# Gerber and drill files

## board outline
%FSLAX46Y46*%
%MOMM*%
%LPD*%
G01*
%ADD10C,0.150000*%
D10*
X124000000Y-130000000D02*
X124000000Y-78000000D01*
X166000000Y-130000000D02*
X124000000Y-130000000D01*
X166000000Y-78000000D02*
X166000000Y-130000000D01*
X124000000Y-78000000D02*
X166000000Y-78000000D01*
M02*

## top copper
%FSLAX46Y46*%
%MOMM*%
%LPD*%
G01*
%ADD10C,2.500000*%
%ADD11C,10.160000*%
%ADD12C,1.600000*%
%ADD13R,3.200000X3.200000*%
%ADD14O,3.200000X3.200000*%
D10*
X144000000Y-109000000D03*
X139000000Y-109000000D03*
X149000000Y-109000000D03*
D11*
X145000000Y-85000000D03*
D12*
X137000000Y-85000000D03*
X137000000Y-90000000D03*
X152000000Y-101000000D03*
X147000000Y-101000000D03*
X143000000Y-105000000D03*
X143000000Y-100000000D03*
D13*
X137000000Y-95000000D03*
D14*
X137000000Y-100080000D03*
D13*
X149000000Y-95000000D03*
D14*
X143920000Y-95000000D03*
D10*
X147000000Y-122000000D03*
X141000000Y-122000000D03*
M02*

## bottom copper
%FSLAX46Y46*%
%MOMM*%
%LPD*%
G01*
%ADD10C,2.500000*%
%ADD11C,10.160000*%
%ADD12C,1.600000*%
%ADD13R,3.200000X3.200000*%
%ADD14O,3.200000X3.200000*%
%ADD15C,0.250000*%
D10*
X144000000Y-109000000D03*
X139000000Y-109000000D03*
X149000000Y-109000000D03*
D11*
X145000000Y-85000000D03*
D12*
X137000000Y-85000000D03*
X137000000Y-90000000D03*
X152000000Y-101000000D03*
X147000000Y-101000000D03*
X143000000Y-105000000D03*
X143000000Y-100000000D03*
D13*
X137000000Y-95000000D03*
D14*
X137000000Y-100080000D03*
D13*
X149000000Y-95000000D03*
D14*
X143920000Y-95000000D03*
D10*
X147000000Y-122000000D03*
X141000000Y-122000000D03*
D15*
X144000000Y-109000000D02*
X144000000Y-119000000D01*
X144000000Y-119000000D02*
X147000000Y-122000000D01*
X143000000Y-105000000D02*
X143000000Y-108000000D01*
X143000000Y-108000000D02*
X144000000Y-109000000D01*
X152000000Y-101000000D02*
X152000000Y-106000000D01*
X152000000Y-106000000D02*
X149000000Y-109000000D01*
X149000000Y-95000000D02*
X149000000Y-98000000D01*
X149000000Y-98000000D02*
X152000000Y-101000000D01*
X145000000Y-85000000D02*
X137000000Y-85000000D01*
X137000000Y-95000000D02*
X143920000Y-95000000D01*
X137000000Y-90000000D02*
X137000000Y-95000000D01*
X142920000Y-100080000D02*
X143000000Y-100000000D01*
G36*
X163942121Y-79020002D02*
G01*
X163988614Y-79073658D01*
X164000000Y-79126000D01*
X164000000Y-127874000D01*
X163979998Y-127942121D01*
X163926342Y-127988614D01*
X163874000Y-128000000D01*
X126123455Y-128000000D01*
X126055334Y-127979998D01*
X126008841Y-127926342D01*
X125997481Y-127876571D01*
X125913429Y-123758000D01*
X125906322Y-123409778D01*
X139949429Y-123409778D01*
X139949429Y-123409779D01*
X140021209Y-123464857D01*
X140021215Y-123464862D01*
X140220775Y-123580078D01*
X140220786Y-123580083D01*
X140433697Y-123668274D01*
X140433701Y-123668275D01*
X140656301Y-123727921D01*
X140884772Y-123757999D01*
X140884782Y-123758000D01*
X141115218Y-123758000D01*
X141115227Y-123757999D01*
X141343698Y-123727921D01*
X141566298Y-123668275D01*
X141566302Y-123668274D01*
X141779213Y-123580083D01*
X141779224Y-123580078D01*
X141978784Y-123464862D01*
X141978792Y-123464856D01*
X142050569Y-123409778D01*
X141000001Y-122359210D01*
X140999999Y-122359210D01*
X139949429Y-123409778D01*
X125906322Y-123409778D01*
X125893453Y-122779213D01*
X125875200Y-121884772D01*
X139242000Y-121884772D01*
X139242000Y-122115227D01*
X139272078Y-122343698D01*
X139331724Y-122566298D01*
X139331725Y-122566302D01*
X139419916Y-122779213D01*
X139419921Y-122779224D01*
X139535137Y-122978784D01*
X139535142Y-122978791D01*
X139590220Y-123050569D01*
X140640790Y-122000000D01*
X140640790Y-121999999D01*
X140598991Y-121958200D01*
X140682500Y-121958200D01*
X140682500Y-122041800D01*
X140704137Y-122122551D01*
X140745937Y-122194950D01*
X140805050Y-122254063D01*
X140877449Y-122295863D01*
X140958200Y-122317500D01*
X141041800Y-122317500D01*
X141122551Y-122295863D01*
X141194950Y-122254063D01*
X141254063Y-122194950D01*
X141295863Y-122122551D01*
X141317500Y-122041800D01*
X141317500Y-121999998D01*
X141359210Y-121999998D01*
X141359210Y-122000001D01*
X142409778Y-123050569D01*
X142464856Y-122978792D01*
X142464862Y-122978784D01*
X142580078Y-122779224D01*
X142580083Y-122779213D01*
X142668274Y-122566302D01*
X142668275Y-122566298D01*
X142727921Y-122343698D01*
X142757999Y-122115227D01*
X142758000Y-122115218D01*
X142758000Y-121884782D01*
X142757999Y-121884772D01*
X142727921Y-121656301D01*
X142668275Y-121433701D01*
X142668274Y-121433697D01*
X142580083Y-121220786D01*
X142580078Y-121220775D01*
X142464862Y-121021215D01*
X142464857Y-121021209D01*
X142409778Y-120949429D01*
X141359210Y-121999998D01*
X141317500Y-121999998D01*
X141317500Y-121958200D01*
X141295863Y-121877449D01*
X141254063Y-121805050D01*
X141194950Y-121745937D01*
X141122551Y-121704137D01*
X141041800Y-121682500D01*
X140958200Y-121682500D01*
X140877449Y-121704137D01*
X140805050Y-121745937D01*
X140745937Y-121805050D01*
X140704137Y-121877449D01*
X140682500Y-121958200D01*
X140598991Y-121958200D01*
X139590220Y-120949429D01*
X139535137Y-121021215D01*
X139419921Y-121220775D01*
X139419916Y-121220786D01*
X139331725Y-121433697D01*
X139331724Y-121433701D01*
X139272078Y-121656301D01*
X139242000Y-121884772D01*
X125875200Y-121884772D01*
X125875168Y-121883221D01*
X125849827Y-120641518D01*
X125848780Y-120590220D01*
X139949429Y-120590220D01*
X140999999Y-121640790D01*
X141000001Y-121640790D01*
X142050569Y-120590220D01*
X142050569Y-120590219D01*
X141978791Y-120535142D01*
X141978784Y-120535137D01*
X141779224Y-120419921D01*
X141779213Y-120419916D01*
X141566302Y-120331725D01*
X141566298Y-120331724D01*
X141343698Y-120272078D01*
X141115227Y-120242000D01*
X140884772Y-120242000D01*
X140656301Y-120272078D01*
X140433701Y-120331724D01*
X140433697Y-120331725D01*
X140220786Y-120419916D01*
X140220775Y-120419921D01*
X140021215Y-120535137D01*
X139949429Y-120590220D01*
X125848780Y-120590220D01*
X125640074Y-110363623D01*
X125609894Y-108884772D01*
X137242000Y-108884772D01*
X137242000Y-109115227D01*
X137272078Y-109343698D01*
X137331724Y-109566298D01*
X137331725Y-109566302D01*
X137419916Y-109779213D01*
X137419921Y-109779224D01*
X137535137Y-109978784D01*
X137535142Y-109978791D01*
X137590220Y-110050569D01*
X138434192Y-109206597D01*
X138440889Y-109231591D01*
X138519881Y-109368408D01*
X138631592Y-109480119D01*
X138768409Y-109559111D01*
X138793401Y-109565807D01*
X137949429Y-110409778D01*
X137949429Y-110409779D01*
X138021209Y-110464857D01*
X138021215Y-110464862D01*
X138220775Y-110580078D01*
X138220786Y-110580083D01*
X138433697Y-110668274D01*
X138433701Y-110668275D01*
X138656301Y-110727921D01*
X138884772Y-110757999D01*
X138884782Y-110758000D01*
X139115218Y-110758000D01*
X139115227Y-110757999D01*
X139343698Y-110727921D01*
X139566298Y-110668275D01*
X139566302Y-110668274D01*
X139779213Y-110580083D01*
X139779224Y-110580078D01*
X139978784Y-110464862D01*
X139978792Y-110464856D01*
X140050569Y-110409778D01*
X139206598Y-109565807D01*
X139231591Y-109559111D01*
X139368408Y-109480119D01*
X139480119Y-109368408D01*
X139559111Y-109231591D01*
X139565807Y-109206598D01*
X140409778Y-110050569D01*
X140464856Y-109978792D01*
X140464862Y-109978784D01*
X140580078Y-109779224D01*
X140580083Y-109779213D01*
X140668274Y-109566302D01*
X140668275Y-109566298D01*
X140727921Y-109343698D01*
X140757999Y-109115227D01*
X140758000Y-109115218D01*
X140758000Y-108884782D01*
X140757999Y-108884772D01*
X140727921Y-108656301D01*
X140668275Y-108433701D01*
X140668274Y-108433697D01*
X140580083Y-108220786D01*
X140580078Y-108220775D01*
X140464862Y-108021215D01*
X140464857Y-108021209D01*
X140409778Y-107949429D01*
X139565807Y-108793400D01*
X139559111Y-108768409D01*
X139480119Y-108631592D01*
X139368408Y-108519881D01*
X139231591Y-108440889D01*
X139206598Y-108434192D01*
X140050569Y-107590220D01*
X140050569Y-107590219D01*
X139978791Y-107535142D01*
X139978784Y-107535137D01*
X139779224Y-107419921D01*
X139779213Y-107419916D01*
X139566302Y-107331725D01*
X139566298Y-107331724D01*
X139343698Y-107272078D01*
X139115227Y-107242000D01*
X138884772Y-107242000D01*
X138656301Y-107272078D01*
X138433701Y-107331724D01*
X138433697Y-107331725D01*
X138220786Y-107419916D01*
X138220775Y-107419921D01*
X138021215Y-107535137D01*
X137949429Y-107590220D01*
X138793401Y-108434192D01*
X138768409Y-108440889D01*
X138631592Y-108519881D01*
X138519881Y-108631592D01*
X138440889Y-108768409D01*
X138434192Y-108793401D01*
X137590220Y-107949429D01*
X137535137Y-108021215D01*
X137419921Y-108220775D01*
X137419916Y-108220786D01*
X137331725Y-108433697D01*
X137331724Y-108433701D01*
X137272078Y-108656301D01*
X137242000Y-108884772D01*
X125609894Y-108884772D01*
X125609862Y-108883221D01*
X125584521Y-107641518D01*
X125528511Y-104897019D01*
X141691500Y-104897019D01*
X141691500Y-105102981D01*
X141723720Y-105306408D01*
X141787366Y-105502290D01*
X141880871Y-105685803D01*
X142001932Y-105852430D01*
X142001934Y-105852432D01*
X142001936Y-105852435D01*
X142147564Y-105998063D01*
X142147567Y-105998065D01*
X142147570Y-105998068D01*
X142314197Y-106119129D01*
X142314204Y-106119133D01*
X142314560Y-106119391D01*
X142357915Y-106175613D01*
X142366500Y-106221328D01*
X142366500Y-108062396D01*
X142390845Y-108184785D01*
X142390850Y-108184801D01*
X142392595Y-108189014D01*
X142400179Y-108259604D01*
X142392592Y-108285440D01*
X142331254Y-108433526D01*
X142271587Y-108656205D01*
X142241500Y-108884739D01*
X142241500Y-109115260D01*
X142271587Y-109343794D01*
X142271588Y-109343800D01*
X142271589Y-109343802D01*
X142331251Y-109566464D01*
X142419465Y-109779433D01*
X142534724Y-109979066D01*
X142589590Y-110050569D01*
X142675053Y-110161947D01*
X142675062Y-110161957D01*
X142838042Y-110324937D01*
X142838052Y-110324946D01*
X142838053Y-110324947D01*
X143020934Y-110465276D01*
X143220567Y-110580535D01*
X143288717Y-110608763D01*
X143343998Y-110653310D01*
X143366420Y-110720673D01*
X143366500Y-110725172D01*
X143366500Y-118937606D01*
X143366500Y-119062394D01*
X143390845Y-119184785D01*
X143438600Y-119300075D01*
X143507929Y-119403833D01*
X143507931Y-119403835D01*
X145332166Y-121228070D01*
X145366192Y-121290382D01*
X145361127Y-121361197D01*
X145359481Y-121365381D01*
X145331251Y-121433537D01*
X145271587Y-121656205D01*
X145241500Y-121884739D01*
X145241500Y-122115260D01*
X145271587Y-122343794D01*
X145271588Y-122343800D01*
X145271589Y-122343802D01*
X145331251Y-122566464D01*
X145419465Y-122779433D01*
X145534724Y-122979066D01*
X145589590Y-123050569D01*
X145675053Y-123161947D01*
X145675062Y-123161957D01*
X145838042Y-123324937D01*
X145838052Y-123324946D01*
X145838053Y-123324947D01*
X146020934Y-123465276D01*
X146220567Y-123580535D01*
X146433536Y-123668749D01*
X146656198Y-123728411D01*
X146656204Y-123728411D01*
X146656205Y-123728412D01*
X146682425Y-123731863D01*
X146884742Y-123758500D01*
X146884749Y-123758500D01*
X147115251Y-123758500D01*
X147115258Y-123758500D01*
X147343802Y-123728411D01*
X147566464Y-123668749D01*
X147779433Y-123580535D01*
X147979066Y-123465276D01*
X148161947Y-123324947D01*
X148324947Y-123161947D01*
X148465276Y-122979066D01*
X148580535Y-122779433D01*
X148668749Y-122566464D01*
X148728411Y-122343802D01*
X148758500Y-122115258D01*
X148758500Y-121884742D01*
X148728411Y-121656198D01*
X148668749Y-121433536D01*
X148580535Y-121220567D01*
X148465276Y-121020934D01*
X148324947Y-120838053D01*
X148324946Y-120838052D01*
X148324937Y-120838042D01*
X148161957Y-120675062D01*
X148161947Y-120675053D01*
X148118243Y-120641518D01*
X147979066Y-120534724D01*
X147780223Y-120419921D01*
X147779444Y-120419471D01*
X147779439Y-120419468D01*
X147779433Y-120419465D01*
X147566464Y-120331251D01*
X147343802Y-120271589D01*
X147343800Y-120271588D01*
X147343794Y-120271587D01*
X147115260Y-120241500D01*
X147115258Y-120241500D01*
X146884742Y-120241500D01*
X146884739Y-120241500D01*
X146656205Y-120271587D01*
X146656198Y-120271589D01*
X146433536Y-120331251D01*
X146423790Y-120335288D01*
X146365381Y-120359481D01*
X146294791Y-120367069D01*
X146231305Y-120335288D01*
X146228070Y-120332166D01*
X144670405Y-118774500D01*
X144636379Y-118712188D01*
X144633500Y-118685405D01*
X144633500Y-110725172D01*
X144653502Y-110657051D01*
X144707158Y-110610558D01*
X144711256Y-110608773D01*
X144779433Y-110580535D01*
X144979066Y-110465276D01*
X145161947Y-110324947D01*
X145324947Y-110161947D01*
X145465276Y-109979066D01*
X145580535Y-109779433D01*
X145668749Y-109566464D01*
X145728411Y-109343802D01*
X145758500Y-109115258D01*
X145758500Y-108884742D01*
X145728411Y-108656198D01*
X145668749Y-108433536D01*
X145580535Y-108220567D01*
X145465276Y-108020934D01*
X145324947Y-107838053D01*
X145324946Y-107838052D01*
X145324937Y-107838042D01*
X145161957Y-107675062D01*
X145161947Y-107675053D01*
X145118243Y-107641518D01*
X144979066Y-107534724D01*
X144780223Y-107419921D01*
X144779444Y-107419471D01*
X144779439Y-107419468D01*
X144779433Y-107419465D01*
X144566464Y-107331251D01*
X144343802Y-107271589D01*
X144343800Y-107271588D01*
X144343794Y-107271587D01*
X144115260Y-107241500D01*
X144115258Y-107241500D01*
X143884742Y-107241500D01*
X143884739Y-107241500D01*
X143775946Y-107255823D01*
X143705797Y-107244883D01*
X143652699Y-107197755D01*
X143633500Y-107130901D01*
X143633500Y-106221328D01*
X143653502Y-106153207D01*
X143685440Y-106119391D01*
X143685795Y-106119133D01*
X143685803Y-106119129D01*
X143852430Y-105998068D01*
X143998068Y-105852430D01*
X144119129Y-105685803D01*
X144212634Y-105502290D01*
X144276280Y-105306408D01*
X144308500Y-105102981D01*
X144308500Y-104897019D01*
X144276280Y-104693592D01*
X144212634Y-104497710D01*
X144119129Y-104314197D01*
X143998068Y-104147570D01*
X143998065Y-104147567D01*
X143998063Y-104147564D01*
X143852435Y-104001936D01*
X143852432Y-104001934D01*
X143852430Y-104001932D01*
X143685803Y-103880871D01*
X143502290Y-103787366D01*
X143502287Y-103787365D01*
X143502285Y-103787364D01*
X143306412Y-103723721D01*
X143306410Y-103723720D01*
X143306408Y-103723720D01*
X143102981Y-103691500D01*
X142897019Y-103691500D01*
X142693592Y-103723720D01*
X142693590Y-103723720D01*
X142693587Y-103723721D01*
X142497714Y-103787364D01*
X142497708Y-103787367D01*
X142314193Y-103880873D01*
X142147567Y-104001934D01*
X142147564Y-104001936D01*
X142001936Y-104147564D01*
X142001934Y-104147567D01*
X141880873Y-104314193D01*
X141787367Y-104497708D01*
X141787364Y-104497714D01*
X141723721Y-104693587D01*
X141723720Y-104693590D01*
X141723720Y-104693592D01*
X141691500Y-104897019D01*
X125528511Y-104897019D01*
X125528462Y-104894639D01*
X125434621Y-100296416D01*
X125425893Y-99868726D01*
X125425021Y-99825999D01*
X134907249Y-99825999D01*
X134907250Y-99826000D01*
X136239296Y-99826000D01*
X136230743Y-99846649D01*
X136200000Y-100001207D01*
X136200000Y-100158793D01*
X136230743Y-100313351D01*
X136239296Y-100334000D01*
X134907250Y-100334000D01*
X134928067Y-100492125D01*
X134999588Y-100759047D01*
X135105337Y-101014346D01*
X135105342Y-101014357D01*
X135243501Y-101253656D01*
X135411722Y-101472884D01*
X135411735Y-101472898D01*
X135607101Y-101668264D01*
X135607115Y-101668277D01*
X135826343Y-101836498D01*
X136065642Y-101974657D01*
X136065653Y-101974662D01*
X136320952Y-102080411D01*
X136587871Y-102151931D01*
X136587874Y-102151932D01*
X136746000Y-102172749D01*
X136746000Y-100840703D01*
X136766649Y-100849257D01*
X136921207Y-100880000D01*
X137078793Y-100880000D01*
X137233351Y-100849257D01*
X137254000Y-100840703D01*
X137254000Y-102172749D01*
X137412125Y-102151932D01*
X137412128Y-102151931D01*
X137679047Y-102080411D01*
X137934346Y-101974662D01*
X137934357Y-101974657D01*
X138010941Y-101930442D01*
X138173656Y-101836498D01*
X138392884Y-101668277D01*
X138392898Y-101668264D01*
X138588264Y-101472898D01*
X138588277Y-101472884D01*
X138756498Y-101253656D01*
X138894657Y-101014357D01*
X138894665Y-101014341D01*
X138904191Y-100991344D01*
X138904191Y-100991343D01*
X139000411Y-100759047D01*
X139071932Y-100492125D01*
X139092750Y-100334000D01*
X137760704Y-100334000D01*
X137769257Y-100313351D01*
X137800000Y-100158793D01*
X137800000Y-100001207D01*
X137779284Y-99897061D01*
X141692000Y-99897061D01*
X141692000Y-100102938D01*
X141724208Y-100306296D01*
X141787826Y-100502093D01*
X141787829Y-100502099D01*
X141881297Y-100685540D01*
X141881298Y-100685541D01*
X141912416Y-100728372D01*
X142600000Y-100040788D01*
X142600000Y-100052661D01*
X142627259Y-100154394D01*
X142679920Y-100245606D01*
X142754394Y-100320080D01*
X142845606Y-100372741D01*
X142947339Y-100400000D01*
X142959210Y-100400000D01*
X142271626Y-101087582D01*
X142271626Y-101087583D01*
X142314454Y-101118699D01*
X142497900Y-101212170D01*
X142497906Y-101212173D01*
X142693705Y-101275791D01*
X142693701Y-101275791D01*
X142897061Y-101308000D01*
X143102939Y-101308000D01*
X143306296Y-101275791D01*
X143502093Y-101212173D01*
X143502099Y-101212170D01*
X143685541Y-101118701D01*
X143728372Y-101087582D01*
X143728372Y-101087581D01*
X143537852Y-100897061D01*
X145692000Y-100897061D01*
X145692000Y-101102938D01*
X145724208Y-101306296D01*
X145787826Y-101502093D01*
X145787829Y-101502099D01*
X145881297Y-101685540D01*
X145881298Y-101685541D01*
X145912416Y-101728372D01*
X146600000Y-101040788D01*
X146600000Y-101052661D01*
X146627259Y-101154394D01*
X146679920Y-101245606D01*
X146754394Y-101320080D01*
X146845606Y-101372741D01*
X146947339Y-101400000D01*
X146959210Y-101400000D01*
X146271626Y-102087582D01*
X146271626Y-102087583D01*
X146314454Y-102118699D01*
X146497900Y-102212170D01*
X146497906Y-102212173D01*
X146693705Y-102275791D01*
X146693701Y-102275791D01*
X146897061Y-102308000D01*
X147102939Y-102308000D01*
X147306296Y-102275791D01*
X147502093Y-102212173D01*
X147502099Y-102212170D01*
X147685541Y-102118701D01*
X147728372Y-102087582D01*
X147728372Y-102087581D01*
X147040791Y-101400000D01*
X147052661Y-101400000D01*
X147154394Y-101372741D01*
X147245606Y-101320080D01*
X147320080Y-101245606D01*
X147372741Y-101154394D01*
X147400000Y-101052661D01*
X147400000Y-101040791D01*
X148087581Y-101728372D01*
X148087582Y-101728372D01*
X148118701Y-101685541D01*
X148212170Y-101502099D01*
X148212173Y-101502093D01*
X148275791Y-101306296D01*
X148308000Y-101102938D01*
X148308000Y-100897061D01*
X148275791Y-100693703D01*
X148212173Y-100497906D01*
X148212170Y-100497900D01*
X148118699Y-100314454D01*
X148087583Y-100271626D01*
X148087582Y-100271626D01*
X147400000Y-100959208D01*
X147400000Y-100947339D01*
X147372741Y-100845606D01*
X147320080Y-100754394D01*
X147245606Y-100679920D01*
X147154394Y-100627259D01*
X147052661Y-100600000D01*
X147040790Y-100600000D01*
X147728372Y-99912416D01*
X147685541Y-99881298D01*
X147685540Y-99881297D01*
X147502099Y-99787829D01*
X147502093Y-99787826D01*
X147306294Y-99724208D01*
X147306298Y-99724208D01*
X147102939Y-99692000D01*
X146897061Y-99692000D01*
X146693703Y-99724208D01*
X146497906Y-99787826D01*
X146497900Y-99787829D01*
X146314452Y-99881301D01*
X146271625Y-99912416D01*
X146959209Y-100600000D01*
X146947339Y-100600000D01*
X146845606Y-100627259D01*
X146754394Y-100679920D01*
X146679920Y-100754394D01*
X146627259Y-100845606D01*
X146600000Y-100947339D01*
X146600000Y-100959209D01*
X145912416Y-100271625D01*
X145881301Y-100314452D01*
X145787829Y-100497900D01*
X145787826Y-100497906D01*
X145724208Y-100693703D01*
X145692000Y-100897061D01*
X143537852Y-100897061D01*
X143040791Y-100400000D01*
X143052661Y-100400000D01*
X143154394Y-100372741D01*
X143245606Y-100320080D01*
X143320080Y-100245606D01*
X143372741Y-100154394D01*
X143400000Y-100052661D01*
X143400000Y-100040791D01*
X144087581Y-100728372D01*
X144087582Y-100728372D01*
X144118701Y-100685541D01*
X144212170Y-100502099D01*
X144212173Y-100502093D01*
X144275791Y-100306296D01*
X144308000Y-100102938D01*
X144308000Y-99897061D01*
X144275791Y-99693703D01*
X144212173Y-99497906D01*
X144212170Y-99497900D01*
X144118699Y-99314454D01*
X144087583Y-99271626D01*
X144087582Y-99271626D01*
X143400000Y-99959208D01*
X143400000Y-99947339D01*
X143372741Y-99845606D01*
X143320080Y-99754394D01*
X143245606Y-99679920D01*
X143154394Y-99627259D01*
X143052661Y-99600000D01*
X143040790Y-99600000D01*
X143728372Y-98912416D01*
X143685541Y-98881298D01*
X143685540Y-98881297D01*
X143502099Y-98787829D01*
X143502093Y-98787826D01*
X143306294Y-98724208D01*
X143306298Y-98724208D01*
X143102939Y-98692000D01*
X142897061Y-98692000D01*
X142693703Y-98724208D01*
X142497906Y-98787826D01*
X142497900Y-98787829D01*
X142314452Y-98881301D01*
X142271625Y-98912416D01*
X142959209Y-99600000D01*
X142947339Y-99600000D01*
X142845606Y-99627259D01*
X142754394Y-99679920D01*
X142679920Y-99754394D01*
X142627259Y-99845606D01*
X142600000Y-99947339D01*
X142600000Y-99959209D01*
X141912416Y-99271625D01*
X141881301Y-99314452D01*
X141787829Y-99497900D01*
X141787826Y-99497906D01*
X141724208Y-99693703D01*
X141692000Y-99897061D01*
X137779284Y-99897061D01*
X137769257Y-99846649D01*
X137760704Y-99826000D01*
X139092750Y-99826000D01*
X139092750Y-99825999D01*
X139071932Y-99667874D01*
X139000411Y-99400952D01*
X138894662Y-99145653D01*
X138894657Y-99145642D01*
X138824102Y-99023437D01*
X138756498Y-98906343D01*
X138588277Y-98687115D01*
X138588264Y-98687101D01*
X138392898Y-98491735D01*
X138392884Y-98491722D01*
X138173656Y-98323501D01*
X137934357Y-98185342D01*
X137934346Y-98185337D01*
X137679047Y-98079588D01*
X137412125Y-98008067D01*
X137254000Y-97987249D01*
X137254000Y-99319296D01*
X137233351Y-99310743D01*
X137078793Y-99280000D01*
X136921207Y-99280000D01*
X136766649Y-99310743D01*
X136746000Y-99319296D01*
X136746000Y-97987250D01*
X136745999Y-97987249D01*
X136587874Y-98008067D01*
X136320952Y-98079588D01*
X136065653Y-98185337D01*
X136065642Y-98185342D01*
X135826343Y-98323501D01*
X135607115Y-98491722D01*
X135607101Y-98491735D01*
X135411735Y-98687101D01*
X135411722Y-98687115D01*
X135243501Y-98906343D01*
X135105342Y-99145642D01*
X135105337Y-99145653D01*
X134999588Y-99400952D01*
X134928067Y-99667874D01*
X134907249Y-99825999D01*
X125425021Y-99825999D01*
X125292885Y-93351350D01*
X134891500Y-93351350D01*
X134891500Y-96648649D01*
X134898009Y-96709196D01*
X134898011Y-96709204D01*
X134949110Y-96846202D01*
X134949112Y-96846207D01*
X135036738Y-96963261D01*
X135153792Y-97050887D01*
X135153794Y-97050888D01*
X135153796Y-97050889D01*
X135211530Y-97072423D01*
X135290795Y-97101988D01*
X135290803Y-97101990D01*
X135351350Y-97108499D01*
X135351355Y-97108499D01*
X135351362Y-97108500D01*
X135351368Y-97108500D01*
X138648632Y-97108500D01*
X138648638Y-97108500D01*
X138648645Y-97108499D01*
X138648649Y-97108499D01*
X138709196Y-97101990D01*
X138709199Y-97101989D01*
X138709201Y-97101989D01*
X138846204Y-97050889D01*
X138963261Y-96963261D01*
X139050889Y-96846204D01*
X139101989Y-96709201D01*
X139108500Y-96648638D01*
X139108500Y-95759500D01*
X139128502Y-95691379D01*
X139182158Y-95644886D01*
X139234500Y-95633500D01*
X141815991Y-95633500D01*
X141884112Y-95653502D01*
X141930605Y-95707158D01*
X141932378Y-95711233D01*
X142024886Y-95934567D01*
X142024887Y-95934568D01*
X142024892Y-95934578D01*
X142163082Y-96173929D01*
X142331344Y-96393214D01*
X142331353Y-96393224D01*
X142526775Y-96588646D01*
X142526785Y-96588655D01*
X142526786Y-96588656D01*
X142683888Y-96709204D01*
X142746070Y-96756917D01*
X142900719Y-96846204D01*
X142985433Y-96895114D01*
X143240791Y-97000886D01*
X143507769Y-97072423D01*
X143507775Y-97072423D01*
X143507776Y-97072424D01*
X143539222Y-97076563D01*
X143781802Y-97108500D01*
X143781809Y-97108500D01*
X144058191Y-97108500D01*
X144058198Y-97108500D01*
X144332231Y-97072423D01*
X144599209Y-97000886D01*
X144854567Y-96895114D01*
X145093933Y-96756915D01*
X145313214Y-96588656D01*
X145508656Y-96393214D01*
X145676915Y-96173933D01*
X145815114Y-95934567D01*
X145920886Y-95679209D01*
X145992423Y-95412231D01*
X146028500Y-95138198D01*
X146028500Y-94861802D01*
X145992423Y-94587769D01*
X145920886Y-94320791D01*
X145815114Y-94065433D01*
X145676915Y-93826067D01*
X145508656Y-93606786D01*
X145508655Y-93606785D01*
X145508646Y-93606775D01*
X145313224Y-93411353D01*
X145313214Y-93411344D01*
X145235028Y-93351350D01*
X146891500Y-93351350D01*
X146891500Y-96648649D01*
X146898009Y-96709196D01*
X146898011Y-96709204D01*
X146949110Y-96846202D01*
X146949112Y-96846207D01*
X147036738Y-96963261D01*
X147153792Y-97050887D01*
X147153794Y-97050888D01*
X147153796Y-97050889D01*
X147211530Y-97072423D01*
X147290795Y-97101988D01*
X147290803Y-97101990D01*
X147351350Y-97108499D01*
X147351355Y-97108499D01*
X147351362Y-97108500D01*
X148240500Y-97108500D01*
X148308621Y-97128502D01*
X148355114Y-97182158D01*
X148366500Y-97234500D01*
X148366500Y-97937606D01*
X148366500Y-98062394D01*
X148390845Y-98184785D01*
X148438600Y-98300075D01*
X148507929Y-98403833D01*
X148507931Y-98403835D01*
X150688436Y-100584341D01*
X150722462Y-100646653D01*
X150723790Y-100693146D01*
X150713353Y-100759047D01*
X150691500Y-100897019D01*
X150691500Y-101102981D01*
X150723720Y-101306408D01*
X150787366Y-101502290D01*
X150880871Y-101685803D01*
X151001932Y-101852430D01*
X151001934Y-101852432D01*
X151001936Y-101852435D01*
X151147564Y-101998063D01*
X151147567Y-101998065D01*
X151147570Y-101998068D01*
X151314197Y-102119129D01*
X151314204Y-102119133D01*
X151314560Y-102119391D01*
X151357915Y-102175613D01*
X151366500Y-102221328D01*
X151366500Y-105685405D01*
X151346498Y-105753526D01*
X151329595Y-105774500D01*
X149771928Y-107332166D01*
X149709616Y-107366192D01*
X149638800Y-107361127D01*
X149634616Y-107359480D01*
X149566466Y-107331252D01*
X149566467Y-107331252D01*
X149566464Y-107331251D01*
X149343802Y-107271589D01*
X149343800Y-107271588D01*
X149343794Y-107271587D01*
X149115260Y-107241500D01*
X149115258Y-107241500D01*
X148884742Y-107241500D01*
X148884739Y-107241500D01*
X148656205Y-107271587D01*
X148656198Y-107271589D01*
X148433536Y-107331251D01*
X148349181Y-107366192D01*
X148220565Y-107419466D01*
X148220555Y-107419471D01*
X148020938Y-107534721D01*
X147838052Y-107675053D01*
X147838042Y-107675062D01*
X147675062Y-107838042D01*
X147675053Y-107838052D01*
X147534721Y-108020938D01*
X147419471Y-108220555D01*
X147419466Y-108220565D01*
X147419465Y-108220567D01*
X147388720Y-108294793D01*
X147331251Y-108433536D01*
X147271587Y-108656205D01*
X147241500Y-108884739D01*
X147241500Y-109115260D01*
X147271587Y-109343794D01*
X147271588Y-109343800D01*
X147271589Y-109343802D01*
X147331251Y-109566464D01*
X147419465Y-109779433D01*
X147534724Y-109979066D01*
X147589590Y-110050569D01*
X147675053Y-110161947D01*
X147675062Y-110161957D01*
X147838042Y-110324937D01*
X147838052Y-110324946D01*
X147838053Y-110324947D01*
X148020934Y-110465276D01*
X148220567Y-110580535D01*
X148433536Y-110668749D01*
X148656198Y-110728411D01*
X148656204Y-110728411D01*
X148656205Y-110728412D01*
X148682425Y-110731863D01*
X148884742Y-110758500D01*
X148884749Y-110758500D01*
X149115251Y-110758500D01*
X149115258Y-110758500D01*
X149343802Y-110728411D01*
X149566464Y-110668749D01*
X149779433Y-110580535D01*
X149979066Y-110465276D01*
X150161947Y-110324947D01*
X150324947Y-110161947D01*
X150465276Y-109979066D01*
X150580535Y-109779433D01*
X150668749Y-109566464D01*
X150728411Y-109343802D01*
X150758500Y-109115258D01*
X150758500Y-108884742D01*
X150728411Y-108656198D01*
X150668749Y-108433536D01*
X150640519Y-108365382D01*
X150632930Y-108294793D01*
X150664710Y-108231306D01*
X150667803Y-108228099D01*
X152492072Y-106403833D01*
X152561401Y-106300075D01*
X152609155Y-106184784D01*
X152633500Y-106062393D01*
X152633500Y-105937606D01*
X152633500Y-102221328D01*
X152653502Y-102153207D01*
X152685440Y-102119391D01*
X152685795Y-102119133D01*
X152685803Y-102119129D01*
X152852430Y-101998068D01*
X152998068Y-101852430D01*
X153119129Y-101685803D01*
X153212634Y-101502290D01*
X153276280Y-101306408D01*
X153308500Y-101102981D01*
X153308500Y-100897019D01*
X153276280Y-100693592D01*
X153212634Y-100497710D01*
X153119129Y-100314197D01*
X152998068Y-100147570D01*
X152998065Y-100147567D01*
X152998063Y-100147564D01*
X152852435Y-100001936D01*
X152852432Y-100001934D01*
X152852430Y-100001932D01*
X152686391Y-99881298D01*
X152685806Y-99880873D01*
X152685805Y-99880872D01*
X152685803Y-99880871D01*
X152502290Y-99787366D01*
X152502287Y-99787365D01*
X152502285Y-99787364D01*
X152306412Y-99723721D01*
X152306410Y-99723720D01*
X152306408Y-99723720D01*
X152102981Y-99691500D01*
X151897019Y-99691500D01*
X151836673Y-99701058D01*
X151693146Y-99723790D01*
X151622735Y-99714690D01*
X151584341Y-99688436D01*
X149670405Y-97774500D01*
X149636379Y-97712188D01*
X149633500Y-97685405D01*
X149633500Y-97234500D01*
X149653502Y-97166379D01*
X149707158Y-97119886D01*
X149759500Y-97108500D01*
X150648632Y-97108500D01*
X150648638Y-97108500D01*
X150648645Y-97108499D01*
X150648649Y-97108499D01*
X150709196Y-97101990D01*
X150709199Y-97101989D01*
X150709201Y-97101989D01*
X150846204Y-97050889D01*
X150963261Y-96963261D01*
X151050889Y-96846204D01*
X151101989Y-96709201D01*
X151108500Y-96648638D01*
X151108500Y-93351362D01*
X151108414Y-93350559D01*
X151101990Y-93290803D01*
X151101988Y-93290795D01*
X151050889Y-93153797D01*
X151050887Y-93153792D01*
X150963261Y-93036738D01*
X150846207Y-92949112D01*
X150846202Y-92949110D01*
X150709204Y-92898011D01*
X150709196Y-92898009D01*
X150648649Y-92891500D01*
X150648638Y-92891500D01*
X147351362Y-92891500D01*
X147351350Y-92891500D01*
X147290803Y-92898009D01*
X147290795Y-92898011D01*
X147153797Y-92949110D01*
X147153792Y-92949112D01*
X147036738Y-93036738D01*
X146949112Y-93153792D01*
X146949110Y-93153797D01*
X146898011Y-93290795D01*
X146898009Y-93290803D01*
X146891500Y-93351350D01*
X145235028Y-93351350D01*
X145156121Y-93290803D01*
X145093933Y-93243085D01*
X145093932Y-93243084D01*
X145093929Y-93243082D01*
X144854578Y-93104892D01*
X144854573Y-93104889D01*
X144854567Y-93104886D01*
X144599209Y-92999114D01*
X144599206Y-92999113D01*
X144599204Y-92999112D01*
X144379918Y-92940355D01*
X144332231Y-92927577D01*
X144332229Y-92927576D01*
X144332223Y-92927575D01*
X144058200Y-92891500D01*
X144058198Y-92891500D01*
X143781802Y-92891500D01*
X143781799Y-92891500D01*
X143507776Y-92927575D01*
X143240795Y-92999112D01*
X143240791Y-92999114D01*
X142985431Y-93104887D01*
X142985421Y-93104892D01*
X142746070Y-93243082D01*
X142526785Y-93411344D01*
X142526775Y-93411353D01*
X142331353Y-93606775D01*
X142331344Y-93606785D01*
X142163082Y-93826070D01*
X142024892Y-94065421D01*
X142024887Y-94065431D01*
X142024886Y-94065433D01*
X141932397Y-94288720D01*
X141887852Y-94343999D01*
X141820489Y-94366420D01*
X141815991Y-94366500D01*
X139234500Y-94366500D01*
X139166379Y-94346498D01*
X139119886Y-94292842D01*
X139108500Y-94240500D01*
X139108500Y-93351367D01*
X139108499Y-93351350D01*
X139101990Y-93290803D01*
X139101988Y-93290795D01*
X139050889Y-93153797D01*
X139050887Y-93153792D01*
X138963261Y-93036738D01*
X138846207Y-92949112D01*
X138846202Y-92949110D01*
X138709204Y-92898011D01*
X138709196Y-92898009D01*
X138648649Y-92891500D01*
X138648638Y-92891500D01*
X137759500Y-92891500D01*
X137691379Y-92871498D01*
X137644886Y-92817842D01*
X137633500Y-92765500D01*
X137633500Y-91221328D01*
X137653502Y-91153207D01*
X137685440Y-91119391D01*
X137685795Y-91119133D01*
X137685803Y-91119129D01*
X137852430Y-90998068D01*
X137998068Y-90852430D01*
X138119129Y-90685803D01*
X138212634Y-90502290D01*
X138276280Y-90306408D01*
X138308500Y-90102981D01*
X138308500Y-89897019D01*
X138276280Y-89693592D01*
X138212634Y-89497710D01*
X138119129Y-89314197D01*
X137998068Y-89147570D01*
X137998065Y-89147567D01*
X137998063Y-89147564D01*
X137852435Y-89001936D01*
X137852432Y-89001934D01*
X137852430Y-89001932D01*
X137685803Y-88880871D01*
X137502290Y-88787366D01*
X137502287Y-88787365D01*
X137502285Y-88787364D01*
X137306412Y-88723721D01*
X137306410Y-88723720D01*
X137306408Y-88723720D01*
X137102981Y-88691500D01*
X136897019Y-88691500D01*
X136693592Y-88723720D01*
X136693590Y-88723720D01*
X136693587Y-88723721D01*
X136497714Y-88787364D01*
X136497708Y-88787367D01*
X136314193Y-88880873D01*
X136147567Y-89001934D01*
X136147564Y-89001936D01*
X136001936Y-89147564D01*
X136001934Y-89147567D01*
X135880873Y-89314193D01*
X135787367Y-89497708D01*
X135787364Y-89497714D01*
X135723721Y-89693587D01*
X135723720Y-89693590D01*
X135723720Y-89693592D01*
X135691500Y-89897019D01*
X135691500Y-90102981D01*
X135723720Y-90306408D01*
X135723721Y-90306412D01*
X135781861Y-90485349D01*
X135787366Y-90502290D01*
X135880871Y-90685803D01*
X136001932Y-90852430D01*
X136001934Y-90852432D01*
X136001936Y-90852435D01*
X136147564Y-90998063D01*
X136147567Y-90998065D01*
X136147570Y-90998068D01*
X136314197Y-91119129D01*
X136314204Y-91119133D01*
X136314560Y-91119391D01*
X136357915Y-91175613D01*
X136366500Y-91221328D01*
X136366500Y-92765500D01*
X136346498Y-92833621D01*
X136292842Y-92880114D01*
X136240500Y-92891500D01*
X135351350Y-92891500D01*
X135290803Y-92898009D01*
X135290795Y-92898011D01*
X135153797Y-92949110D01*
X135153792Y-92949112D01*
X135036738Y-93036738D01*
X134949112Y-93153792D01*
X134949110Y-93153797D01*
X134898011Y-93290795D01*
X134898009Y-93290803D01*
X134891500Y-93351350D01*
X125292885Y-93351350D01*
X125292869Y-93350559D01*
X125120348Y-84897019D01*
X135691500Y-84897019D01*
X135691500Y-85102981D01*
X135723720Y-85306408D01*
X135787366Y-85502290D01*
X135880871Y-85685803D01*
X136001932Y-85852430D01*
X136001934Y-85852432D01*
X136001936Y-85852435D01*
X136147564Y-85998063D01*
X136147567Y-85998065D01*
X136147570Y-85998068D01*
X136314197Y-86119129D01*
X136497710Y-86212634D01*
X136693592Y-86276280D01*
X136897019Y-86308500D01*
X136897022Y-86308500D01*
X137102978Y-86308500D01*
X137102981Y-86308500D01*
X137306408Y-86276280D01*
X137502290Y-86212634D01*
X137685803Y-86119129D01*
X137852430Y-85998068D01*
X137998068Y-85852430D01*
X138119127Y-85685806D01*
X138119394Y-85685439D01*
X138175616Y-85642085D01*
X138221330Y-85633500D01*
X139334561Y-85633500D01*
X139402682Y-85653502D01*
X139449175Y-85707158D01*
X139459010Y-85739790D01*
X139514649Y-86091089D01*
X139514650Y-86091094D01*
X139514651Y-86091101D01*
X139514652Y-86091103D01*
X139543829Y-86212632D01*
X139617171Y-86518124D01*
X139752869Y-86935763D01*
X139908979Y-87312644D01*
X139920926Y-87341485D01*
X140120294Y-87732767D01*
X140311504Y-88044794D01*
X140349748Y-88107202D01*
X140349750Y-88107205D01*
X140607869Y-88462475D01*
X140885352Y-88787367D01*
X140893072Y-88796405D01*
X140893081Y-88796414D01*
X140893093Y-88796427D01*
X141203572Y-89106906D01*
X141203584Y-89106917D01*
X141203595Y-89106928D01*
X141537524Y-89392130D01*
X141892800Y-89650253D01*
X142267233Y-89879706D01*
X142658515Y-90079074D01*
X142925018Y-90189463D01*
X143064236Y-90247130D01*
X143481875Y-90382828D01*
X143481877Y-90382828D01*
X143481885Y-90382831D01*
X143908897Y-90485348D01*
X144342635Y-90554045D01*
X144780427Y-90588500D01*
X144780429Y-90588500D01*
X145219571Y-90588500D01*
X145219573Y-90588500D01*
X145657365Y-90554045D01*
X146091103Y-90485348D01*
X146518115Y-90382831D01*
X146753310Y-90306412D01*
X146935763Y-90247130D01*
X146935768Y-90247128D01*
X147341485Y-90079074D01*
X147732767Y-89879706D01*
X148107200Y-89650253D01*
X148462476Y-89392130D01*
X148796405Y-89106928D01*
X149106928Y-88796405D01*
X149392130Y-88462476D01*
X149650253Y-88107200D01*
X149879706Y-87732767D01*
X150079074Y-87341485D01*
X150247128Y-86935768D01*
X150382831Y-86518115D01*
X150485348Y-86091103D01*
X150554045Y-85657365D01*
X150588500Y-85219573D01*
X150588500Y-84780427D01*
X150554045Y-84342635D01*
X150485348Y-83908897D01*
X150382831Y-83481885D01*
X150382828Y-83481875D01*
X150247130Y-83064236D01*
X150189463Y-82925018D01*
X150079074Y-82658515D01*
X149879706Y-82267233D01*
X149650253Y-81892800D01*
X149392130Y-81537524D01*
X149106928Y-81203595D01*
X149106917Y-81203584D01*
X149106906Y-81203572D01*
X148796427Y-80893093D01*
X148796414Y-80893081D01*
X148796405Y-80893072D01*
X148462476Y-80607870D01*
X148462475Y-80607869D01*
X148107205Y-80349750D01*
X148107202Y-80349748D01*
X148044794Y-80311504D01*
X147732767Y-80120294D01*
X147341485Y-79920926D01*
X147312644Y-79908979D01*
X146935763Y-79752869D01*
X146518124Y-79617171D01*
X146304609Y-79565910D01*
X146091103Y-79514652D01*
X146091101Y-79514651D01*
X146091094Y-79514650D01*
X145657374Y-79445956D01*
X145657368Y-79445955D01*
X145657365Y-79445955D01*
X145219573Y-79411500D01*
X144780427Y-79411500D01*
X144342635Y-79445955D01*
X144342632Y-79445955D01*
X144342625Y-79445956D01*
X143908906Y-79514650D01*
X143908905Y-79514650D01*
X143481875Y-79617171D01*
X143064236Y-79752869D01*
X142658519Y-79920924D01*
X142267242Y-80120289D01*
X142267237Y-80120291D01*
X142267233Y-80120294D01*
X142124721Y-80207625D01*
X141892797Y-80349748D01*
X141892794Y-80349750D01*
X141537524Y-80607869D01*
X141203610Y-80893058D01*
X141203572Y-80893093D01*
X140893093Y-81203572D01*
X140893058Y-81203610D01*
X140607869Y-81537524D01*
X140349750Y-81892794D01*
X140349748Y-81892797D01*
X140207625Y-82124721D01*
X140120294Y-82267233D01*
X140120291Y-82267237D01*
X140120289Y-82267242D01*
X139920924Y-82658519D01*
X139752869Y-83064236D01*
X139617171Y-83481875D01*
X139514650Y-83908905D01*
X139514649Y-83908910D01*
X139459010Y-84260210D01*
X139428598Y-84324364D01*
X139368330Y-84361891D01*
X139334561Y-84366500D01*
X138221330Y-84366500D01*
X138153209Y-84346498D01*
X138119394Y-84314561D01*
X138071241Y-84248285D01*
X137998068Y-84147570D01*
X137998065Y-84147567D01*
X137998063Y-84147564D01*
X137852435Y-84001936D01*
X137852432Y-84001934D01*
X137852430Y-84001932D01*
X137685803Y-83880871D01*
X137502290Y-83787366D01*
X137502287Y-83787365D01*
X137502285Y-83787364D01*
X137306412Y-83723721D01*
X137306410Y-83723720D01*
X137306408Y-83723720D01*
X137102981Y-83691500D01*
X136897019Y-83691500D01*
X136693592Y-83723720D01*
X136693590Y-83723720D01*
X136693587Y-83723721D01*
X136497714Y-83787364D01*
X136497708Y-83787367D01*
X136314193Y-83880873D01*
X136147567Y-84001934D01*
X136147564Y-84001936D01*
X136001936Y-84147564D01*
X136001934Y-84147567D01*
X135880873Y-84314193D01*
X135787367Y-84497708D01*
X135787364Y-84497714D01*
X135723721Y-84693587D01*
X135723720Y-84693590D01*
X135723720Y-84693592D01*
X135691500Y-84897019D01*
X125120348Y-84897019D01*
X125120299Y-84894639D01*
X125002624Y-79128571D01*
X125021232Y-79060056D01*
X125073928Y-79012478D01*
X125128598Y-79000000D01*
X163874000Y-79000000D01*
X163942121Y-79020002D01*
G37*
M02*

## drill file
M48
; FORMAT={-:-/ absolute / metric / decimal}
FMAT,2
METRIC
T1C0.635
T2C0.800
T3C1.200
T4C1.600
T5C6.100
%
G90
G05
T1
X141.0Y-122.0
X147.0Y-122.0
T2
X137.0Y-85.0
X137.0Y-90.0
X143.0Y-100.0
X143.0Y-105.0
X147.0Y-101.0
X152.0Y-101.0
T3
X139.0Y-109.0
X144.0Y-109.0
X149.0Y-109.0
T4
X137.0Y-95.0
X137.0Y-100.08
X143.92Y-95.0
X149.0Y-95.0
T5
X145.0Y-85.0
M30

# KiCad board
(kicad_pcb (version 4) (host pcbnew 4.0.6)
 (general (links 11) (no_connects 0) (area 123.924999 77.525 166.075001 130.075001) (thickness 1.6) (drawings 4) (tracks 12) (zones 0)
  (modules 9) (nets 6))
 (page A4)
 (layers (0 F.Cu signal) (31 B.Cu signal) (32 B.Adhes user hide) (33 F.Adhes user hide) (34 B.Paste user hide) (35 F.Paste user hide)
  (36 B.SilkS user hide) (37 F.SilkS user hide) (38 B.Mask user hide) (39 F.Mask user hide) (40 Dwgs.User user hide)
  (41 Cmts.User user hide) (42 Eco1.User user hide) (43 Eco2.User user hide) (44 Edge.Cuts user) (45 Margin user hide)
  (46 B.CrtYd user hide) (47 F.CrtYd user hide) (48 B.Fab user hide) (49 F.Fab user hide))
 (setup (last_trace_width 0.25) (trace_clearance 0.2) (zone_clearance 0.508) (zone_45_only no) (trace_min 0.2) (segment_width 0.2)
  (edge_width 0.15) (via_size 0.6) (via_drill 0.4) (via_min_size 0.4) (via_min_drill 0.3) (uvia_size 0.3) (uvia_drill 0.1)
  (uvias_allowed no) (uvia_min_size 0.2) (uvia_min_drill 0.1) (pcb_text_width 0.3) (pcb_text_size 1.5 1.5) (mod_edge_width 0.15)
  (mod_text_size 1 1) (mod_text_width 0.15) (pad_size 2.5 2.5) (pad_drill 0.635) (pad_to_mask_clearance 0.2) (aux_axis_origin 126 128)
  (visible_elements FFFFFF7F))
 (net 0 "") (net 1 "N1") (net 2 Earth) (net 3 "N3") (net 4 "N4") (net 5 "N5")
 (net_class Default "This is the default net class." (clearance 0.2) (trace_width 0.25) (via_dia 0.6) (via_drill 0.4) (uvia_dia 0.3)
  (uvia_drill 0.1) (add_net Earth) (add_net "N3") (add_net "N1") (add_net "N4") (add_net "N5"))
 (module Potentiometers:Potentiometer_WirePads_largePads (layer F.Cu) (at 149 109 270)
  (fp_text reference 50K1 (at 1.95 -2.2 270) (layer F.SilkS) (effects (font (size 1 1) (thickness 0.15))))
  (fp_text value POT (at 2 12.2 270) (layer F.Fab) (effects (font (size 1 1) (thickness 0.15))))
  (pad 2 thru_hole circle (at 0 5 270) (size 2.5 2.5) (drill 1.2) (layers *.Cu *.Mask) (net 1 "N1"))
  (pad 3 thru_hole circle (at 0 10 270) (size 2.5 2.5) (drill 1.2) (layers *.Cu *.Mask) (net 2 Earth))
  (pad 1 thru_hole circle (at 0 0 270) (size 2.5 2.5) (drill 1.2) (layers *.Cu *.Mask) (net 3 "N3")))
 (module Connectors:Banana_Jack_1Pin (layer F.Cu) (at 145 85)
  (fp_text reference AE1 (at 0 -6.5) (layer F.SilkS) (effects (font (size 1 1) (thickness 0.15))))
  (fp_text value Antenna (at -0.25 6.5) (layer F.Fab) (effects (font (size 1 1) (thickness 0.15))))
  (pad 1 thru_hole circle (at 0 0) (size 10.16 10.16) (drill 6.1) (layers *.Cu *.Mask) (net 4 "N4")))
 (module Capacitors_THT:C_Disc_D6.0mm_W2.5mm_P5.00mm (layer F.Cu) (at 137 85 270)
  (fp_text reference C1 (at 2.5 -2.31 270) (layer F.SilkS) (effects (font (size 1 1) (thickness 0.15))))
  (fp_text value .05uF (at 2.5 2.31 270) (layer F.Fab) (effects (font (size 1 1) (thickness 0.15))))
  (pad 1 thru_hole circle (at 0 0 270) (size 1.6 1.6) (drill 0.8) (layers *.Cu *.Mask) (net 4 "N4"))
  (pad 2 thru_hole circle (at 5 0 270) (size 1.6 1.6) (drill 0.8) (layers *.Cu *.Mask) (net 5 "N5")))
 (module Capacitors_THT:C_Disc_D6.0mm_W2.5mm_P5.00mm (layer F.Cu) (at 152 101 180)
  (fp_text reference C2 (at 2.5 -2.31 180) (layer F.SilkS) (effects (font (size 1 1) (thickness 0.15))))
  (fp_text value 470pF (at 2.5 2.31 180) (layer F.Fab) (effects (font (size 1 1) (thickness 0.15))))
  (pad 1 thru_hole circle (at 0 0 180) (size 1.6 1.6) (drill 0.8) (layers *.Cu *.Mask) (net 3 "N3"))
  (pad 2 thru_hole circle (at 5 0 180) (size 1.6 1.6) (drill 0.8) (layers *.Cu *.Mask) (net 2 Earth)))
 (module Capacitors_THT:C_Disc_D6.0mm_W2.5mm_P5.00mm (layer F.Cu) (at 143 105 90)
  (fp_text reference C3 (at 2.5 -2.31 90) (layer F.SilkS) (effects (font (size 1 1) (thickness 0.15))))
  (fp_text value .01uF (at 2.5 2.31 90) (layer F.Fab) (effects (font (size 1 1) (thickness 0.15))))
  (pad 1 thru_hole circle (at 0 0 90) (size 1.6 1.6) (drill 0.8) (layers *.Cu *.Mask) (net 1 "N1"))
  (pad 2 thru_hole circle (at 5 0 90) (size 1.6 1.6) (drill 0.8) (layers *.Cu *.Mask) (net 2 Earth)))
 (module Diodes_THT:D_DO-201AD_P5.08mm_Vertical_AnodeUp (layer F.Cu) (at 137 95 270)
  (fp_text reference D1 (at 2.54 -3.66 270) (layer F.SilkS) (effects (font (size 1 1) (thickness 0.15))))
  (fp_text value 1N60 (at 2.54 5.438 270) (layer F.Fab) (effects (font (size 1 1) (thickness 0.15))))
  (pad 1 thru_hole rect (at 0 0 270) (size 3.2 3.2) (drill 1.6) (layers *.Cu *.Mask) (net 5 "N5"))
  (pad 2 thru_hole oval (at 5.08 0 270) (size 3.2 3.2) (drill 1.6) (layers *.Cu *.Mask) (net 2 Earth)))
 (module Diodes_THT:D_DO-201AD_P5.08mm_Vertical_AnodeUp (layer F.Cu) (at 149 95 180)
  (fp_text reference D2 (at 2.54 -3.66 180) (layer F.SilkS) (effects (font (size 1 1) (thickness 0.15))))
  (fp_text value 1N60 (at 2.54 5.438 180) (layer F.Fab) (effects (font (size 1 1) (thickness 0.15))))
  (pad 1 thru_hole rect (at 0 0 180) (size 3.2 3.2) (drill 1.6) (layers *.Cu *.Mask) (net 3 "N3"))
  (pad 2 thru_hole oval (at 5.08 0 180) (size 3.2 3.2) (drill 1.6) (layers *.Cu *.Mask) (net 5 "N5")))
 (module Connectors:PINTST (layer F.Cu) (at 147 122)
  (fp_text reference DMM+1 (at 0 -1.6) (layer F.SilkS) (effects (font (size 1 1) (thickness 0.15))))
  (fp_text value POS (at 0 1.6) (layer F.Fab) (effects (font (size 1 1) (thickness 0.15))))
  (pad 1 thru_hole circle (at 0 0) (size 2.5 2.5) (drill 0.635) (layers *.Cu *.Mask) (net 1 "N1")))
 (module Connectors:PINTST (layer F.Cu) (at 141 122)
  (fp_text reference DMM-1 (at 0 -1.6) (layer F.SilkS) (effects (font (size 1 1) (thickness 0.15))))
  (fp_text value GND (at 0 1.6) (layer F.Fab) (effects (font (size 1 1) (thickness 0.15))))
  (pad 1 thru_hole circle (at 0 0) (size 2.5 2.5) (drill 0.635) (layers *.Cu *.Mask) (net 2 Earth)))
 (gr_line (start 124 130) (end 124 78) (angle 90) (layer Edge.Cuts) (width 0.15))
 (gr_line (start 166 130) (end 124 130) (angle 90) (layer Edge.Cuts) (width 0.15))
 (gr_line (start 166 78) (end 166 130) (angle 90) (layer Edge.Cuts) (width 0.15))
 (gr_line (start 124 78) (end 166 78) (angle 90) (layer Edge.Cuts) (width 0.15))
 (segment (start 144 109) (end 144 119) (width 0.25) (layer B.Cu) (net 1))
 (segment (start 144 119) (end 147 122) (width 0.25) (layer B.Cu) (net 1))
 (segment (start 143 105) (end 143 108) (width 0.25) (layer B.Cu) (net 1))
 (segment (start 143 108) (end 144 109) (width 0.25) (layer B.Cu) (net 1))
 (segment (start 152 101) (end 152 106) (width 0.25) (layer B.Cu) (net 3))
 (segment (start 152 106) (end 149 109) (width 0.25) (layer B.Cu) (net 3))
 (segment (start 149 95) (end 149 98) (width 0.25) (layer B.Cu) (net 3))
 (segment (start 149 98) (end 152 101) (width 0.25) (layer B.Cu) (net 3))
 (segment (start 145 85) (end 137 85) (width 0.25) (layer B.Cu) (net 4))
 (segment (start 137 95) (end 143.92 95) (width 0.25) (layer B.Cu) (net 5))
 (segment (start 137 90) (end 137 95) (width 0.25) (layer B.Cu) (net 5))
 (segment (start 142.92 100.08) (end 143 100) (width 0.25) (layer B.Cu) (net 2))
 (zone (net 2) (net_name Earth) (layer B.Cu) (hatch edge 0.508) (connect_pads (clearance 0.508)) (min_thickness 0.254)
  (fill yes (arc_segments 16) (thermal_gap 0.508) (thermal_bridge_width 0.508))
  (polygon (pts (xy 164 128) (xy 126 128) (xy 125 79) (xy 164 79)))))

